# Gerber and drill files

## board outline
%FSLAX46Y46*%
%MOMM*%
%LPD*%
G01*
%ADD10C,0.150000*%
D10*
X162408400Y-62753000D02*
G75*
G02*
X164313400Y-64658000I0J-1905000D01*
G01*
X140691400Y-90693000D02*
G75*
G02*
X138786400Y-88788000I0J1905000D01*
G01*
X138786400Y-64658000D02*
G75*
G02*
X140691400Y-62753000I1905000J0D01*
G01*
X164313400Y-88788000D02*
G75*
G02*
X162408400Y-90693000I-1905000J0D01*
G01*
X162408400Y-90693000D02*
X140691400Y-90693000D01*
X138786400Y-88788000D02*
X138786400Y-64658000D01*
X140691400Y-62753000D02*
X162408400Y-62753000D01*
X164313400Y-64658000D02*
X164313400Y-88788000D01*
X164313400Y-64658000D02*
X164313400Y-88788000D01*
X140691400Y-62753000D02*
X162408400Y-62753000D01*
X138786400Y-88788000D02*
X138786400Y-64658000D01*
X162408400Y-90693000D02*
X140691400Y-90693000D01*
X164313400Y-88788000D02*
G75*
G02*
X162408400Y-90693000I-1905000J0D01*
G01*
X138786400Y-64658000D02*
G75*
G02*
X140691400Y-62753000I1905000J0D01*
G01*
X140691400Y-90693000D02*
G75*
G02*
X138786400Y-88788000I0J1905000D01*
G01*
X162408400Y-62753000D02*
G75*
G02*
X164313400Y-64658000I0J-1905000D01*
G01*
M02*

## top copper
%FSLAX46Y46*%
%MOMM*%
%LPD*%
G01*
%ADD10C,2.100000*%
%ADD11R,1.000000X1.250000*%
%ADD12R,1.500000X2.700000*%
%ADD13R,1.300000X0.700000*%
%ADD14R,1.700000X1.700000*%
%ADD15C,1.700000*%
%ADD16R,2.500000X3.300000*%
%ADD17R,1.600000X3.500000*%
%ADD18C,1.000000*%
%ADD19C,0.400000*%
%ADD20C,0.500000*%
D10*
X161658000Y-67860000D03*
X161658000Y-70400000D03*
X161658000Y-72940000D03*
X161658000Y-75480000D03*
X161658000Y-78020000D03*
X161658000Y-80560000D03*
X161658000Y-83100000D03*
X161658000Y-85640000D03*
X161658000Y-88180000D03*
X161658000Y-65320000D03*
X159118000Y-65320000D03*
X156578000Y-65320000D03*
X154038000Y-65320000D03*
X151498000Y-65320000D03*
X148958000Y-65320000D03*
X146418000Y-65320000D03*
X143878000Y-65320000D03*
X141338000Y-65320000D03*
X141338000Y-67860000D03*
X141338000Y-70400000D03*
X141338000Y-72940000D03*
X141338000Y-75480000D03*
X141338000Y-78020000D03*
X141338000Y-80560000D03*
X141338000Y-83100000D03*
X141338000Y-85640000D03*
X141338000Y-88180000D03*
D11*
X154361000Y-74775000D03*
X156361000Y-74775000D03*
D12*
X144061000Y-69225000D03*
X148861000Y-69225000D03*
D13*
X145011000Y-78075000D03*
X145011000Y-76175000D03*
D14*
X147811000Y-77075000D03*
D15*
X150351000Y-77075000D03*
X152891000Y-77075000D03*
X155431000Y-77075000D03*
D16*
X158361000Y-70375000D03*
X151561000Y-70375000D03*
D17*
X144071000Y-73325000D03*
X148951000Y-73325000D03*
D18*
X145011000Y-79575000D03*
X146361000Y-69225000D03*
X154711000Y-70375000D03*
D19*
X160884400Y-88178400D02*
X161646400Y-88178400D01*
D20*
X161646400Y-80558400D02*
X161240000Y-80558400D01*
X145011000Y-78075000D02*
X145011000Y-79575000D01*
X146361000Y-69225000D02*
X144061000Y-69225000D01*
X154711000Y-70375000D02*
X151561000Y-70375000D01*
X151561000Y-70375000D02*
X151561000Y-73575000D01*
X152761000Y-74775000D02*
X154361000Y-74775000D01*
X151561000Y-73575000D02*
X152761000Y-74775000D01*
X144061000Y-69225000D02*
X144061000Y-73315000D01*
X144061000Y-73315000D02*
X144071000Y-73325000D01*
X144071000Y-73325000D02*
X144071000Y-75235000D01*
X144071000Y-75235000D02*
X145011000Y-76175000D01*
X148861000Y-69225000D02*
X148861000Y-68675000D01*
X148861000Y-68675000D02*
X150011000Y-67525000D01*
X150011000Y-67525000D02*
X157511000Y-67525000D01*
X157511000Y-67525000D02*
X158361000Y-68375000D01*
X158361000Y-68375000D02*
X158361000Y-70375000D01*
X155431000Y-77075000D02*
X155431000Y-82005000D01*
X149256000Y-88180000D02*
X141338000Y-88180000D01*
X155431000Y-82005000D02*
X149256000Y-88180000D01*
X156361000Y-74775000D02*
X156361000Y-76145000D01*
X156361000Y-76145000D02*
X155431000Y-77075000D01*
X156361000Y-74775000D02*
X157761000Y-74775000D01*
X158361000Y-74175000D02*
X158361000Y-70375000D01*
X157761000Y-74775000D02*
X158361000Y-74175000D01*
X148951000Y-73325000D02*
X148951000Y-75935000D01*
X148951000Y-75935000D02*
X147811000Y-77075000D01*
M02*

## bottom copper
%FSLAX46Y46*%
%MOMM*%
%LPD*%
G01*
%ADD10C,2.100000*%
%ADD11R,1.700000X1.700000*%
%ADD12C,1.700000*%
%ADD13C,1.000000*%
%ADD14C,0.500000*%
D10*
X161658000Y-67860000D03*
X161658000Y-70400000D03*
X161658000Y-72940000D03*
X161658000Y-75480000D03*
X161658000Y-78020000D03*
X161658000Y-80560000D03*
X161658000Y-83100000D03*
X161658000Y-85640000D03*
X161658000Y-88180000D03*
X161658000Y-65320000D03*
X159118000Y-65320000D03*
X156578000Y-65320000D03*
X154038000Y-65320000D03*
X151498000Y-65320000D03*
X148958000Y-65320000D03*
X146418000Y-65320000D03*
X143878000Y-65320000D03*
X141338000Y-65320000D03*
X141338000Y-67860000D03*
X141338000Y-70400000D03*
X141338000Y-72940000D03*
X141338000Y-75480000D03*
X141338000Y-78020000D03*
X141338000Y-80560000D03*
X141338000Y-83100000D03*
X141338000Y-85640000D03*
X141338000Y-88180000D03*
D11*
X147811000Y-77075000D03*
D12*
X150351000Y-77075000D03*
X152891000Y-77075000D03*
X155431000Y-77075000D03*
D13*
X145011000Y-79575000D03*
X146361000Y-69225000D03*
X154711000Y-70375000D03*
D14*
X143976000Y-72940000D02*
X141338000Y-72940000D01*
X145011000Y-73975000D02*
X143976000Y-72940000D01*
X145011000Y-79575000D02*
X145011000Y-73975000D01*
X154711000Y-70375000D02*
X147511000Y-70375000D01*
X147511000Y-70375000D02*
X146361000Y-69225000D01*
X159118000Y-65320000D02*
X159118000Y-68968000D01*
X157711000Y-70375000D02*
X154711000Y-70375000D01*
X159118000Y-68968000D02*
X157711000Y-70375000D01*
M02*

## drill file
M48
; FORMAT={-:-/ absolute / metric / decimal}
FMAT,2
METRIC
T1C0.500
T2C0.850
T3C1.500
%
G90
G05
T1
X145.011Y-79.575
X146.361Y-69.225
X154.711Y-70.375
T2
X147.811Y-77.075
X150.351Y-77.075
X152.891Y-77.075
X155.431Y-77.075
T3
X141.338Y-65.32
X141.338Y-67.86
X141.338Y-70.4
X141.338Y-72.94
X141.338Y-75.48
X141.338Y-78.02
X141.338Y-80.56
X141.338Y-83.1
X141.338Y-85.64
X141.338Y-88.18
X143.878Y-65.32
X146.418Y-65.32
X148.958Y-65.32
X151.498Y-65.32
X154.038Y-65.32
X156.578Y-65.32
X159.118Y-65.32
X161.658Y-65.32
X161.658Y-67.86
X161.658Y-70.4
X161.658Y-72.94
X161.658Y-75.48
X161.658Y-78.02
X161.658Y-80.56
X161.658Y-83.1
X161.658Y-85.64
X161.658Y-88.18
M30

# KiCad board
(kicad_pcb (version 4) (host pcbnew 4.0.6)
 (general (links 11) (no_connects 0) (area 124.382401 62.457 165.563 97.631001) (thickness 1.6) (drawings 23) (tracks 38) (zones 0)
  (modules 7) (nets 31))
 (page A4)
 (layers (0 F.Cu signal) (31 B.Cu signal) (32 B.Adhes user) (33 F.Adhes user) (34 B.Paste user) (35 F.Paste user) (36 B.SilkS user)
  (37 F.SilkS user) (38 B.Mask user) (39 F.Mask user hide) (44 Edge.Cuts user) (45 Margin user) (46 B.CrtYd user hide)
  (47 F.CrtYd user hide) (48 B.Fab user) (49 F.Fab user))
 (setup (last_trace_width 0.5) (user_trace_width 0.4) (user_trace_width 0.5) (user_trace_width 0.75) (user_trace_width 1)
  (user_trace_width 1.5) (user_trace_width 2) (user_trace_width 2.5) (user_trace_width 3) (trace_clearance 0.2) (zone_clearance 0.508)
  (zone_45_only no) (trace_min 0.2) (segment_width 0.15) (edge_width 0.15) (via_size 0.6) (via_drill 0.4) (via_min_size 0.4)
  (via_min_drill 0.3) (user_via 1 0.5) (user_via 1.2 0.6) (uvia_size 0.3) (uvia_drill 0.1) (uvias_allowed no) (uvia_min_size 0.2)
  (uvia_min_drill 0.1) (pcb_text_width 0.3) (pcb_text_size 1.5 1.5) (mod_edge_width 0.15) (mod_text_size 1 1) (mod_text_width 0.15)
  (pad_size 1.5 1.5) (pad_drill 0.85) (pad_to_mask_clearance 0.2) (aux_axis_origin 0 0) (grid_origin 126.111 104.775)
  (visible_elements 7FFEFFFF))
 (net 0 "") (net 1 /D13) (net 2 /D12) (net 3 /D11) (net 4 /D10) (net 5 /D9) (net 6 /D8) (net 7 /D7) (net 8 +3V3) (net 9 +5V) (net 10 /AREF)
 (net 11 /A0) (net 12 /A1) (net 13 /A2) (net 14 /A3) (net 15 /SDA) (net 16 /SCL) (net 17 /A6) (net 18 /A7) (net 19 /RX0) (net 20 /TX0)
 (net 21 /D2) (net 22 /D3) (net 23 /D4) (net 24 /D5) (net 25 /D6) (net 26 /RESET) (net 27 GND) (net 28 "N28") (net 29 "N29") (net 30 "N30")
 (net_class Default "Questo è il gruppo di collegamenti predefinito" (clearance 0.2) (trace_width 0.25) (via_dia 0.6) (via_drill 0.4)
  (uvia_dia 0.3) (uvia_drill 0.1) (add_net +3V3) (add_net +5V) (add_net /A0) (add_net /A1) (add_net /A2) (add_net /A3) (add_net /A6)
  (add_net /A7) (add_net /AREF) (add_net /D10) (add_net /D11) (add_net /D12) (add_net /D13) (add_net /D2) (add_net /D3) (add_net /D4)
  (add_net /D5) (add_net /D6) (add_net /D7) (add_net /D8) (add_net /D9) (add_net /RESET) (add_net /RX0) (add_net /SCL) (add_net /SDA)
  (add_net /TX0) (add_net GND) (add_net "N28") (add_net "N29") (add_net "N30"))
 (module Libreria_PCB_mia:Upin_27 (layer B.Cu) (at 161.658 88.18 180)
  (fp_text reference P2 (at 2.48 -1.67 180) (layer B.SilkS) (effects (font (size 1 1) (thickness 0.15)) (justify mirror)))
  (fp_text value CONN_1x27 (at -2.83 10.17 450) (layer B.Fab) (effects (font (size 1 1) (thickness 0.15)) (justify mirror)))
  (pad 9 thru_hole circle (at 0 20.32 180) (size 2.1 2.1) (drill 1.5) (layers *.Cu *.Mask) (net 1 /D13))
  (pad 8 thru_hole circle (at 0 17.78 180) (size 2.1 2.1) (drill 1.5) (layers *.Cu *.Mask) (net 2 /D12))
  (pad 7 thru_hole circle (at 0 15.24 180) (size 2.1 2.1) (drill 1.5) (layers *.Cu *.Mask) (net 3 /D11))
  (pad 6 thru_hole circle (at 0 12.7 180) (size 2.1 2.1) (drill 1.5) (layers *.Cu *.Mask) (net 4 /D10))
  (pad 5 thru_hole circle (at 0 10.16 180) (size 2.1 2.1) (drill 1.5) (layers *.Cu *.Mask) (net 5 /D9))
  (pad 4 thru_hole circle (at 0 7.62 180) (size 2.1 2.1) (drill 1.5) (layers *.Cu *.Mask) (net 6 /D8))
  (pad 3 thru_hole circle (at 0 5.08 180) (size 2.1 2.1) (drill 1.5) (layers *.Cu *.Mask) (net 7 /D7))
  (pad 2 thru_hole circle (at 0 2.54 180) (size 2.1 2.1) (drill 1.5) (layers *.Cu *.Mask) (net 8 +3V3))
  (pad 1 thru_hole circle (at 0 0 180) (size 2.1 2.1) (drill 1.5) (layers *.Cu *.Mask) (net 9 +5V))
  (pad 10 thru_hole circle (at 0 22.86 180) (size 2.1 2.1) (drill 1.5) (layers *.Cu *.Mask) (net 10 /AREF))
  (pad 11 thru_hole circle (at 2.54 22.86 180) (size 2.1 2.1) (drill 1.5) (layers *.Cu *.Mask) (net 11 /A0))
  (pad 12 thru_hole circle (at 5.08 22.86 180) (size 2.1 2.1) (drill 1.5) (layers *.Cu *.Mask) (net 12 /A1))
  (pad 13 thru_hole circle (at 7.62 22.86 180) (size 2.1 2.1) (drill 1.5) (layers *.Cu *.Mask) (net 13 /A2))
  (pad 14 thru_hole circle (at 10.16 22.86 180) (size 2.1 2.1) (drill 1.5) (layers *.Cu *.Mask) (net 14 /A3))
  (pad 15 thru_hole circle (at 12.7 22.86 180) (size 2.1 2.1) (drill 1.5) (layers *.Cu *.Mask) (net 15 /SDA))
  (pad 16 thru_hole circle (at 15.24 22.86 180) (size 2.1 2.1) (drill 1.5) (layers *.Cu *.Mask) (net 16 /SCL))
  (pad 17 thru_hole circle (at 17.78 22.86 180) (size 2.1 2.1) (drill 1.5) (layers *.Cu *.Mask) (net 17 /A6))
  (pad 18 thru_hole circle (at 20.32 22.86 180) (size 2.1 2.1) (drill 1.5) (layers *.Cu *.Mask) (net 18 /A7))
  (pad 19 thru_hole circle (at 20.32 20.32 180) (size 2.1 2.1) (drill 1.5) (layers *.Cu *.Mask) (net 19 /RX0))
  (pad 20 thru_hole circle (at 20.32 17.78 180) (size 2.1 2.1) (drill 1.5) (layers *.Cu *.Mask) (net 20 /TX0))
  (pad 21 thru_hole circle (at 20.32 15.24 180) (size 2.1 2.1) (drill 1.5) (layers *.Cu *.Mask) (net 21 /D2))
  (pad 22 thru_hole circle (at 20.32 12.7 180) (size 2.1 2.1) (drill 1.5) (layers *.Cu *.Mask) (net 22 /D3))
  (pad 23 thru_hole circle (at 20.32 10.16 180) (size 2.1 2.1) (drill 1.5) (layers *.Cu *.Mask) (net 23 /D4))
  (pad 24 thru_hole circle (at 20.32 7.62 180) (size 2.1 2.1) (drill 1.5) (layers *.Cu *.Mask) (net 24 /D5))
  (pad 25 thru_hole circle (at 20.32 5.08 180) (size 2.1 2.1) (drill 1.5) (layers *.Cu *.Mask) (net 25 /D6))
  (pad 26 thru_hole circle (at 20.32 2.54 180) (size 2.1 2.1) (drill 1.5) (layers *.Cu *.Mask) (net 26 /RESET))
  (pad 27 thru_hole circle (at 20.32 0 180) (size 2.1 2.1) (drill 1.5) (layers *.Cu *.Mask) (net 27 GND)))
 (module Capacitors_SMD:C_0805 (layer F.Cu) (at 155.361 74.775)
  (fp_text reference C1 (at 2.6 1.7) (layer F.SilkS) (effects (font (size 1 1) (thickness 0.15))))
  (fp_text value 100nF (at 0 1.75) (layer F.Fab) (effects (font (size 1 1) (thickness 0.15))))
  (pad 1 smd rect (at -1 0) (size 1 1.25) (layers F.Cu F.Paste F.Mask) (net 11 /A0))
  (pad 2 smd rect (at 1 0) (size 1 1.25) (layers F.Cu F.Paste F.Mask) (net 27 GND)))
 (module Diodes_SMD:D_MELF (layer F.Cu) (at 146.461 69.225)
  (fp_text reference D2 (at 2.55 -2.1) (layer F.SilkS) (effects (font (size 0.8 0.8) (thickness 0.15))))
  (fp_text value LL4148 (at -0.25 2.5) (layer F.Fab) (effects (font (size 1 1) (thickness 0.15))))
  (pad 1 smd rect (at -2.4 0) (size 1.5 2.7) (layers F.Cu F.Paste F.Mask) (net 11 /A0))
  (pad 2 smd rect (at 2.4 0) (size 1.5 2.7) (layers F.Cu F.Paste F.Mask) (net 27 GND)))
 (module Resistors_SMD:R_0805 (layer F.Cu) (at 145.011 77.125 90)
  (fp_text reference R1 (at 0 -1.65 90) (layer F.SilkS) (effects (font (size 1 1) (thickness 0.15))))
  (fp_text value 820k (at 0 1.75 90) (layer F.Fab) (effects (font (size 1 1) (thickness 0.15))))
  (pad 1 smd rect (at -0.95 0 90) (size 0.7 1.3) (layers F.Cu F.Paste F.Mask) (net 21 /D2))
  (pad 2 smd rect (at 0.95 0 90) (size 0.7 1.3) (layers F.Cu F.Paste F.Mask) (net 11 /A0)))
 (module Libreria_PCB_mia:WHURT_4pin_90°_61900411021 (layer F.Cu) (at 147.811 77.075)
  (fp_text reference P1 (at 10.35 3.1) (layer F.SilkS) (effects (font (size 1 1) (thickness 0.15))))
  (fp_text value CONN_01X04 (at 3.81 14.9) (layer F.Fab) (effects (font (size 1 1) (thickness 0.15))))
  (pad 1 thru_hole rect (at 0 0) (size 1.7 1.7) (drill 0.85) (layers *.Cu *.Mask) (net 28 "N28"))
  (pad 2 thru_hole circle (at 2.54 0) (size 1.7 1.7) (drill 0.85) (layers *.Cu *.Mask) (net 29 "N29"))
  (pad 3 thru_hole circle (at 5.08 0) (size 1.7 1.7) (drill 0.85) (layers *.Cu *.Mask) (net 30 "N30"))
  (pad 4 thru_hole circle (at 7.62 0) (size 1.7 1.7) (drill 0.85) (layers *.Cu *.Mask) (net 27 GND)))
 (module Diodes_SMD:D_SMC (layer F.Cu) (at 154.961 70.375 180)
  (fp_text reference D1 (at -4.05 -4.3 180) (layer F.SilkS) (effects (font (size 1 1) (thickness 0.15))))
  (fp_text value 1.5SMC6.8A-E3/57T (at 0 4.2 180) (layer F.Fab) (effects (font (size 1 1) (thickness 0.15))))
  (pad 1 smd rect (at -3.4 0 270) (size 3.3 2.5) (layers F.Cu F.Paste F.Mask) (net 27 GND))
  (pad 2 smd rect (at 3.4 0 270) (size 3.3 2.5) (layers F.Cu F.Paste F.Mask) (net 11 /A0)))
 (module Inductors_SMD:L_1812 (layer F.Cu) (at 146.511 73.325)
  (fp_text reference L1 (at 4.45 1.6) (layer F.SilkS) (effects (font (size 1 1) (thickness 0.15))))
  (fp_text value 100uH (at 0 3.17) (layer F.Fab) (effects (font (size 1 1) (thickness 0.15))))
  (pad 1 smd rect (at -2.44 0) (size 1.6 3.5) (layers F.Cu F.Paste F.Mask) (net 11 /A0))
  (pad 2 smd rect (at 2.44 0) (size 1.6 3.5) (layers F.Cu F.Paste F.Mask) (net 28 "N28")))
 (gr_arc (start 162.4084 64.658) (end 162.4084 62.753) (angle 90) (layer Edge.Cuts) (width 0.15))
 (gr_arc (start 140.6914 88.788) (end 140.6914 90.693) (angle 90) (layer Edge.Cuts) (width 0.15))
 (gr_arc (start 140.6914 64.658) (end 138.7864 64.658) (angle 90) (layer Edge.Cuts) (width 0.15))
 (gr_arc (start 162.4084 88.788) (end 164.3134 88.788) (angle 90) (layer Edge.Cuts) (width 0.15))
 (gr_line (start 162.4084 90.693) (end 140.6914 90.693) (angle 90) (layer Edge.Cuts) (width 0.15))
 (gr_line (start 138.7864 88.788) (end 138.7864 64.658) (angle 90) (layer Edge.Cuts) (width 0.15))
 (gr_line (start 140.6914 62.753) (end 162.4084 62.753) (angle 90) (layer Edge.Cuts) (width 0.15))
 (gr_line (start 164.3134 64.658) (end 164.3134 88.788) (angle 90) (layer Edge.Cuts) (width 0.15))
 (gr_line (start 164.3134 64.658) (end 164.3134 88.788) (angle 90) (layer Edge.Cuts) (width 0.15))
 (gr_line (start 140.6914 62.753) (end 162.4084 62.753) (angle 90) (layer Edge.Cuts) (width 0.15))
 (gr_line (start 138.7864 88.788) (end 138.7864 64.658) (angle 90) (layer Edge.Cuts) (width 0.15))
 (gr_line (start 162.4084 90.693) (end 140.6914 90.693) (angle 90) (layer Edge.Cuts) (width 0.15))
 (gr_arc (start 162.4084 88.788) (end 164.3134 88.788) (angle 90) (layer Edge.Cuts) (width 0.15))
 (gr_arc (start 140.6914 64.658) (end 138.7864 64.658) (angle 90) (layer Edge.Cuts) (width 0.15))
 (gr_arc (start 140.6914 88.788) (end 140.6914 90.693) (angle 90) (layer Edge.Cuts) (width 0.15))
 (gr_arc (start 162.4084 64.658) (end 162.4084 62.753) (angle 90) (layer Edge.Cuts) (width 0.15))
 (segment (start 160.8844 88.1784) (end 161.6464 88.1784) (width 0.4) (layer F.Cu) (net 9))
 (segment (start 161.6464 80.5584) (end 161.24 80.5584) (width 0.5) (layer F.Cu) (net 6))
 (segment (start 145.011 78.075) (end 145.011 79.575) (width 0.5) (layer F.Cu) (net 21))
 (segment (start 143.976 72.94) (end 141.338 72.94) (width 0.5) (layer B.Cu) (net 21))
 (segment (start 145.011 73.975) (end 143.976 72.94) (width 0.5) (layer B.Cu) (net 21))
 (segment (start 145.011 79.575) (end 145.011 73.975) (width 0.5) (layer B.Cu) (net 21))
 (via (at 145.011 79.575) (size 1) (drill 0.5) (layers F.Cu B.Cu) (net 21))
 (segment (start 154.711 70.375) (end 147.511 70.375) (width 0.5) (layer B.Cu) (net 11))
 (segment (start 146.361 69.225) (end 144.061 69.225) (width 0.5) (layer F.Cu) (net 11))
 (via (at 146.361 69.225) (size 1) (drill 0.5) (layers F.Cu B.Cu) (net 11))
 (segment (start 147.511 70.375) (end 146.361 69.225) (width 0.5) (layer B.Cu) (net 11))
 (segment (start 159.118 65.32) (end 159.118 68.968) (width 0.5) (layer B.Cu) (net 11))
 (segment (start 154.711 70.375) (end 151.561 70.375) (width 0.5) (layer F.Cu) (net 11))
 (via (at 154.711 70.375) (size 1) (drill 0.5) (layers F.Cu B.Cu) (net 11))
 (segment (start 157.711 70.375) (end 154.711 70.375) (width 0.5) (layer B.Cu) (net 11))
 (segment (start 159.118 68.968) (end 157.711 70.375) (width 0.5) (layer B.Cu) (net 11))
 (segment (start 151.561 70.375) (end 151.561 73.575) (width 0.5) (layer F.Cu) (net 11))
 (segment (start 152.761 74.775) (end 154.361 74.775) (width 0.5) (layer F.Cu) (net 11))
 (segment (start 151.561 73.575) (end 152.761 74.775) (width 0.5) (layer F.Cu) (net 11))
 (segment (start 144.061 69.225) (end 144.061 73.315) (width 0.5) (layer F.Cu) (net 11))
 (segment (start 144.061 73.315) (end 144.071 73.325) (width 0.5) (layer F.Cu) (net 11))
 (segment (start 144.071 73.325) (end 144.071 75.235) (width 0.5) (layer F.Cu) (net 11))
 (segment (start 144.071 75.235) (end 145.011 76.175) (width 0.5) (layer F.Cu) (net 11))
 (segment (start 148.861 69.225) (end 148.861 68.675) (width 0.5) (layer F.Cu) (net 27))
 (segment (start 148.861 68.675) (end 150.011 67.525) (width 0.5) (layer F.Cu) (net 27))
 (segment (start 150.011 67.525) (end 157.511 67.525) (width 0.5) (layer F.Cu) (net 27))
 (segment (start 157.511 67.525) (end 158.361 68.375) (width 0.5) (layer F.Cu) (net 27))
 (segment (start 158.361 68.375) (end 158.361 70.375) (width 0.5) (layer F.Cu) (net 27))
 (segment (start 155.431 77.075) (end 155.431 82.005) (width 0.5) (layer F.Cu) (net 27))
 (segment (start 149.256 88.18) (end 141.338 88.18) (width 0.5) (layer F.Cu) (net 27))
 (segment (start 155.431 82.005) (end 149.256 88.18) (width 0.5) (layer F.Cu) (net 27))
 (segment (start 156.361 74.775) (end 156.361 76.145) (width 0.5) (layer F.Cu) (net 27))
 (segment (start 156.361 76.145) (end 155.431 77.075) (width 0.5) (layer F.Cu) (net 27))
 (segment (start 156.361 74.775) (end 157.761 74.775) (width 0.5) (layer F.Cu) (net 27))
 (segment (start 158.361 74.175) (end 158.361 70.375) (width 0.5) (layer F.Cu) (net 27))
 (segment (start 157.761 74.775) (end 158.361 74.175) (width 0.5) (layer F.Cu) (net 27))
 (segment (start 148.951 73.325) (end 148.951 75.935) (width 0.5) (layer F.Cu) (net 28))
 (segment (start 148.951 75.935) (end 147.811 77.075) (width 0.5) (layer F.Cu) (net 28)))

